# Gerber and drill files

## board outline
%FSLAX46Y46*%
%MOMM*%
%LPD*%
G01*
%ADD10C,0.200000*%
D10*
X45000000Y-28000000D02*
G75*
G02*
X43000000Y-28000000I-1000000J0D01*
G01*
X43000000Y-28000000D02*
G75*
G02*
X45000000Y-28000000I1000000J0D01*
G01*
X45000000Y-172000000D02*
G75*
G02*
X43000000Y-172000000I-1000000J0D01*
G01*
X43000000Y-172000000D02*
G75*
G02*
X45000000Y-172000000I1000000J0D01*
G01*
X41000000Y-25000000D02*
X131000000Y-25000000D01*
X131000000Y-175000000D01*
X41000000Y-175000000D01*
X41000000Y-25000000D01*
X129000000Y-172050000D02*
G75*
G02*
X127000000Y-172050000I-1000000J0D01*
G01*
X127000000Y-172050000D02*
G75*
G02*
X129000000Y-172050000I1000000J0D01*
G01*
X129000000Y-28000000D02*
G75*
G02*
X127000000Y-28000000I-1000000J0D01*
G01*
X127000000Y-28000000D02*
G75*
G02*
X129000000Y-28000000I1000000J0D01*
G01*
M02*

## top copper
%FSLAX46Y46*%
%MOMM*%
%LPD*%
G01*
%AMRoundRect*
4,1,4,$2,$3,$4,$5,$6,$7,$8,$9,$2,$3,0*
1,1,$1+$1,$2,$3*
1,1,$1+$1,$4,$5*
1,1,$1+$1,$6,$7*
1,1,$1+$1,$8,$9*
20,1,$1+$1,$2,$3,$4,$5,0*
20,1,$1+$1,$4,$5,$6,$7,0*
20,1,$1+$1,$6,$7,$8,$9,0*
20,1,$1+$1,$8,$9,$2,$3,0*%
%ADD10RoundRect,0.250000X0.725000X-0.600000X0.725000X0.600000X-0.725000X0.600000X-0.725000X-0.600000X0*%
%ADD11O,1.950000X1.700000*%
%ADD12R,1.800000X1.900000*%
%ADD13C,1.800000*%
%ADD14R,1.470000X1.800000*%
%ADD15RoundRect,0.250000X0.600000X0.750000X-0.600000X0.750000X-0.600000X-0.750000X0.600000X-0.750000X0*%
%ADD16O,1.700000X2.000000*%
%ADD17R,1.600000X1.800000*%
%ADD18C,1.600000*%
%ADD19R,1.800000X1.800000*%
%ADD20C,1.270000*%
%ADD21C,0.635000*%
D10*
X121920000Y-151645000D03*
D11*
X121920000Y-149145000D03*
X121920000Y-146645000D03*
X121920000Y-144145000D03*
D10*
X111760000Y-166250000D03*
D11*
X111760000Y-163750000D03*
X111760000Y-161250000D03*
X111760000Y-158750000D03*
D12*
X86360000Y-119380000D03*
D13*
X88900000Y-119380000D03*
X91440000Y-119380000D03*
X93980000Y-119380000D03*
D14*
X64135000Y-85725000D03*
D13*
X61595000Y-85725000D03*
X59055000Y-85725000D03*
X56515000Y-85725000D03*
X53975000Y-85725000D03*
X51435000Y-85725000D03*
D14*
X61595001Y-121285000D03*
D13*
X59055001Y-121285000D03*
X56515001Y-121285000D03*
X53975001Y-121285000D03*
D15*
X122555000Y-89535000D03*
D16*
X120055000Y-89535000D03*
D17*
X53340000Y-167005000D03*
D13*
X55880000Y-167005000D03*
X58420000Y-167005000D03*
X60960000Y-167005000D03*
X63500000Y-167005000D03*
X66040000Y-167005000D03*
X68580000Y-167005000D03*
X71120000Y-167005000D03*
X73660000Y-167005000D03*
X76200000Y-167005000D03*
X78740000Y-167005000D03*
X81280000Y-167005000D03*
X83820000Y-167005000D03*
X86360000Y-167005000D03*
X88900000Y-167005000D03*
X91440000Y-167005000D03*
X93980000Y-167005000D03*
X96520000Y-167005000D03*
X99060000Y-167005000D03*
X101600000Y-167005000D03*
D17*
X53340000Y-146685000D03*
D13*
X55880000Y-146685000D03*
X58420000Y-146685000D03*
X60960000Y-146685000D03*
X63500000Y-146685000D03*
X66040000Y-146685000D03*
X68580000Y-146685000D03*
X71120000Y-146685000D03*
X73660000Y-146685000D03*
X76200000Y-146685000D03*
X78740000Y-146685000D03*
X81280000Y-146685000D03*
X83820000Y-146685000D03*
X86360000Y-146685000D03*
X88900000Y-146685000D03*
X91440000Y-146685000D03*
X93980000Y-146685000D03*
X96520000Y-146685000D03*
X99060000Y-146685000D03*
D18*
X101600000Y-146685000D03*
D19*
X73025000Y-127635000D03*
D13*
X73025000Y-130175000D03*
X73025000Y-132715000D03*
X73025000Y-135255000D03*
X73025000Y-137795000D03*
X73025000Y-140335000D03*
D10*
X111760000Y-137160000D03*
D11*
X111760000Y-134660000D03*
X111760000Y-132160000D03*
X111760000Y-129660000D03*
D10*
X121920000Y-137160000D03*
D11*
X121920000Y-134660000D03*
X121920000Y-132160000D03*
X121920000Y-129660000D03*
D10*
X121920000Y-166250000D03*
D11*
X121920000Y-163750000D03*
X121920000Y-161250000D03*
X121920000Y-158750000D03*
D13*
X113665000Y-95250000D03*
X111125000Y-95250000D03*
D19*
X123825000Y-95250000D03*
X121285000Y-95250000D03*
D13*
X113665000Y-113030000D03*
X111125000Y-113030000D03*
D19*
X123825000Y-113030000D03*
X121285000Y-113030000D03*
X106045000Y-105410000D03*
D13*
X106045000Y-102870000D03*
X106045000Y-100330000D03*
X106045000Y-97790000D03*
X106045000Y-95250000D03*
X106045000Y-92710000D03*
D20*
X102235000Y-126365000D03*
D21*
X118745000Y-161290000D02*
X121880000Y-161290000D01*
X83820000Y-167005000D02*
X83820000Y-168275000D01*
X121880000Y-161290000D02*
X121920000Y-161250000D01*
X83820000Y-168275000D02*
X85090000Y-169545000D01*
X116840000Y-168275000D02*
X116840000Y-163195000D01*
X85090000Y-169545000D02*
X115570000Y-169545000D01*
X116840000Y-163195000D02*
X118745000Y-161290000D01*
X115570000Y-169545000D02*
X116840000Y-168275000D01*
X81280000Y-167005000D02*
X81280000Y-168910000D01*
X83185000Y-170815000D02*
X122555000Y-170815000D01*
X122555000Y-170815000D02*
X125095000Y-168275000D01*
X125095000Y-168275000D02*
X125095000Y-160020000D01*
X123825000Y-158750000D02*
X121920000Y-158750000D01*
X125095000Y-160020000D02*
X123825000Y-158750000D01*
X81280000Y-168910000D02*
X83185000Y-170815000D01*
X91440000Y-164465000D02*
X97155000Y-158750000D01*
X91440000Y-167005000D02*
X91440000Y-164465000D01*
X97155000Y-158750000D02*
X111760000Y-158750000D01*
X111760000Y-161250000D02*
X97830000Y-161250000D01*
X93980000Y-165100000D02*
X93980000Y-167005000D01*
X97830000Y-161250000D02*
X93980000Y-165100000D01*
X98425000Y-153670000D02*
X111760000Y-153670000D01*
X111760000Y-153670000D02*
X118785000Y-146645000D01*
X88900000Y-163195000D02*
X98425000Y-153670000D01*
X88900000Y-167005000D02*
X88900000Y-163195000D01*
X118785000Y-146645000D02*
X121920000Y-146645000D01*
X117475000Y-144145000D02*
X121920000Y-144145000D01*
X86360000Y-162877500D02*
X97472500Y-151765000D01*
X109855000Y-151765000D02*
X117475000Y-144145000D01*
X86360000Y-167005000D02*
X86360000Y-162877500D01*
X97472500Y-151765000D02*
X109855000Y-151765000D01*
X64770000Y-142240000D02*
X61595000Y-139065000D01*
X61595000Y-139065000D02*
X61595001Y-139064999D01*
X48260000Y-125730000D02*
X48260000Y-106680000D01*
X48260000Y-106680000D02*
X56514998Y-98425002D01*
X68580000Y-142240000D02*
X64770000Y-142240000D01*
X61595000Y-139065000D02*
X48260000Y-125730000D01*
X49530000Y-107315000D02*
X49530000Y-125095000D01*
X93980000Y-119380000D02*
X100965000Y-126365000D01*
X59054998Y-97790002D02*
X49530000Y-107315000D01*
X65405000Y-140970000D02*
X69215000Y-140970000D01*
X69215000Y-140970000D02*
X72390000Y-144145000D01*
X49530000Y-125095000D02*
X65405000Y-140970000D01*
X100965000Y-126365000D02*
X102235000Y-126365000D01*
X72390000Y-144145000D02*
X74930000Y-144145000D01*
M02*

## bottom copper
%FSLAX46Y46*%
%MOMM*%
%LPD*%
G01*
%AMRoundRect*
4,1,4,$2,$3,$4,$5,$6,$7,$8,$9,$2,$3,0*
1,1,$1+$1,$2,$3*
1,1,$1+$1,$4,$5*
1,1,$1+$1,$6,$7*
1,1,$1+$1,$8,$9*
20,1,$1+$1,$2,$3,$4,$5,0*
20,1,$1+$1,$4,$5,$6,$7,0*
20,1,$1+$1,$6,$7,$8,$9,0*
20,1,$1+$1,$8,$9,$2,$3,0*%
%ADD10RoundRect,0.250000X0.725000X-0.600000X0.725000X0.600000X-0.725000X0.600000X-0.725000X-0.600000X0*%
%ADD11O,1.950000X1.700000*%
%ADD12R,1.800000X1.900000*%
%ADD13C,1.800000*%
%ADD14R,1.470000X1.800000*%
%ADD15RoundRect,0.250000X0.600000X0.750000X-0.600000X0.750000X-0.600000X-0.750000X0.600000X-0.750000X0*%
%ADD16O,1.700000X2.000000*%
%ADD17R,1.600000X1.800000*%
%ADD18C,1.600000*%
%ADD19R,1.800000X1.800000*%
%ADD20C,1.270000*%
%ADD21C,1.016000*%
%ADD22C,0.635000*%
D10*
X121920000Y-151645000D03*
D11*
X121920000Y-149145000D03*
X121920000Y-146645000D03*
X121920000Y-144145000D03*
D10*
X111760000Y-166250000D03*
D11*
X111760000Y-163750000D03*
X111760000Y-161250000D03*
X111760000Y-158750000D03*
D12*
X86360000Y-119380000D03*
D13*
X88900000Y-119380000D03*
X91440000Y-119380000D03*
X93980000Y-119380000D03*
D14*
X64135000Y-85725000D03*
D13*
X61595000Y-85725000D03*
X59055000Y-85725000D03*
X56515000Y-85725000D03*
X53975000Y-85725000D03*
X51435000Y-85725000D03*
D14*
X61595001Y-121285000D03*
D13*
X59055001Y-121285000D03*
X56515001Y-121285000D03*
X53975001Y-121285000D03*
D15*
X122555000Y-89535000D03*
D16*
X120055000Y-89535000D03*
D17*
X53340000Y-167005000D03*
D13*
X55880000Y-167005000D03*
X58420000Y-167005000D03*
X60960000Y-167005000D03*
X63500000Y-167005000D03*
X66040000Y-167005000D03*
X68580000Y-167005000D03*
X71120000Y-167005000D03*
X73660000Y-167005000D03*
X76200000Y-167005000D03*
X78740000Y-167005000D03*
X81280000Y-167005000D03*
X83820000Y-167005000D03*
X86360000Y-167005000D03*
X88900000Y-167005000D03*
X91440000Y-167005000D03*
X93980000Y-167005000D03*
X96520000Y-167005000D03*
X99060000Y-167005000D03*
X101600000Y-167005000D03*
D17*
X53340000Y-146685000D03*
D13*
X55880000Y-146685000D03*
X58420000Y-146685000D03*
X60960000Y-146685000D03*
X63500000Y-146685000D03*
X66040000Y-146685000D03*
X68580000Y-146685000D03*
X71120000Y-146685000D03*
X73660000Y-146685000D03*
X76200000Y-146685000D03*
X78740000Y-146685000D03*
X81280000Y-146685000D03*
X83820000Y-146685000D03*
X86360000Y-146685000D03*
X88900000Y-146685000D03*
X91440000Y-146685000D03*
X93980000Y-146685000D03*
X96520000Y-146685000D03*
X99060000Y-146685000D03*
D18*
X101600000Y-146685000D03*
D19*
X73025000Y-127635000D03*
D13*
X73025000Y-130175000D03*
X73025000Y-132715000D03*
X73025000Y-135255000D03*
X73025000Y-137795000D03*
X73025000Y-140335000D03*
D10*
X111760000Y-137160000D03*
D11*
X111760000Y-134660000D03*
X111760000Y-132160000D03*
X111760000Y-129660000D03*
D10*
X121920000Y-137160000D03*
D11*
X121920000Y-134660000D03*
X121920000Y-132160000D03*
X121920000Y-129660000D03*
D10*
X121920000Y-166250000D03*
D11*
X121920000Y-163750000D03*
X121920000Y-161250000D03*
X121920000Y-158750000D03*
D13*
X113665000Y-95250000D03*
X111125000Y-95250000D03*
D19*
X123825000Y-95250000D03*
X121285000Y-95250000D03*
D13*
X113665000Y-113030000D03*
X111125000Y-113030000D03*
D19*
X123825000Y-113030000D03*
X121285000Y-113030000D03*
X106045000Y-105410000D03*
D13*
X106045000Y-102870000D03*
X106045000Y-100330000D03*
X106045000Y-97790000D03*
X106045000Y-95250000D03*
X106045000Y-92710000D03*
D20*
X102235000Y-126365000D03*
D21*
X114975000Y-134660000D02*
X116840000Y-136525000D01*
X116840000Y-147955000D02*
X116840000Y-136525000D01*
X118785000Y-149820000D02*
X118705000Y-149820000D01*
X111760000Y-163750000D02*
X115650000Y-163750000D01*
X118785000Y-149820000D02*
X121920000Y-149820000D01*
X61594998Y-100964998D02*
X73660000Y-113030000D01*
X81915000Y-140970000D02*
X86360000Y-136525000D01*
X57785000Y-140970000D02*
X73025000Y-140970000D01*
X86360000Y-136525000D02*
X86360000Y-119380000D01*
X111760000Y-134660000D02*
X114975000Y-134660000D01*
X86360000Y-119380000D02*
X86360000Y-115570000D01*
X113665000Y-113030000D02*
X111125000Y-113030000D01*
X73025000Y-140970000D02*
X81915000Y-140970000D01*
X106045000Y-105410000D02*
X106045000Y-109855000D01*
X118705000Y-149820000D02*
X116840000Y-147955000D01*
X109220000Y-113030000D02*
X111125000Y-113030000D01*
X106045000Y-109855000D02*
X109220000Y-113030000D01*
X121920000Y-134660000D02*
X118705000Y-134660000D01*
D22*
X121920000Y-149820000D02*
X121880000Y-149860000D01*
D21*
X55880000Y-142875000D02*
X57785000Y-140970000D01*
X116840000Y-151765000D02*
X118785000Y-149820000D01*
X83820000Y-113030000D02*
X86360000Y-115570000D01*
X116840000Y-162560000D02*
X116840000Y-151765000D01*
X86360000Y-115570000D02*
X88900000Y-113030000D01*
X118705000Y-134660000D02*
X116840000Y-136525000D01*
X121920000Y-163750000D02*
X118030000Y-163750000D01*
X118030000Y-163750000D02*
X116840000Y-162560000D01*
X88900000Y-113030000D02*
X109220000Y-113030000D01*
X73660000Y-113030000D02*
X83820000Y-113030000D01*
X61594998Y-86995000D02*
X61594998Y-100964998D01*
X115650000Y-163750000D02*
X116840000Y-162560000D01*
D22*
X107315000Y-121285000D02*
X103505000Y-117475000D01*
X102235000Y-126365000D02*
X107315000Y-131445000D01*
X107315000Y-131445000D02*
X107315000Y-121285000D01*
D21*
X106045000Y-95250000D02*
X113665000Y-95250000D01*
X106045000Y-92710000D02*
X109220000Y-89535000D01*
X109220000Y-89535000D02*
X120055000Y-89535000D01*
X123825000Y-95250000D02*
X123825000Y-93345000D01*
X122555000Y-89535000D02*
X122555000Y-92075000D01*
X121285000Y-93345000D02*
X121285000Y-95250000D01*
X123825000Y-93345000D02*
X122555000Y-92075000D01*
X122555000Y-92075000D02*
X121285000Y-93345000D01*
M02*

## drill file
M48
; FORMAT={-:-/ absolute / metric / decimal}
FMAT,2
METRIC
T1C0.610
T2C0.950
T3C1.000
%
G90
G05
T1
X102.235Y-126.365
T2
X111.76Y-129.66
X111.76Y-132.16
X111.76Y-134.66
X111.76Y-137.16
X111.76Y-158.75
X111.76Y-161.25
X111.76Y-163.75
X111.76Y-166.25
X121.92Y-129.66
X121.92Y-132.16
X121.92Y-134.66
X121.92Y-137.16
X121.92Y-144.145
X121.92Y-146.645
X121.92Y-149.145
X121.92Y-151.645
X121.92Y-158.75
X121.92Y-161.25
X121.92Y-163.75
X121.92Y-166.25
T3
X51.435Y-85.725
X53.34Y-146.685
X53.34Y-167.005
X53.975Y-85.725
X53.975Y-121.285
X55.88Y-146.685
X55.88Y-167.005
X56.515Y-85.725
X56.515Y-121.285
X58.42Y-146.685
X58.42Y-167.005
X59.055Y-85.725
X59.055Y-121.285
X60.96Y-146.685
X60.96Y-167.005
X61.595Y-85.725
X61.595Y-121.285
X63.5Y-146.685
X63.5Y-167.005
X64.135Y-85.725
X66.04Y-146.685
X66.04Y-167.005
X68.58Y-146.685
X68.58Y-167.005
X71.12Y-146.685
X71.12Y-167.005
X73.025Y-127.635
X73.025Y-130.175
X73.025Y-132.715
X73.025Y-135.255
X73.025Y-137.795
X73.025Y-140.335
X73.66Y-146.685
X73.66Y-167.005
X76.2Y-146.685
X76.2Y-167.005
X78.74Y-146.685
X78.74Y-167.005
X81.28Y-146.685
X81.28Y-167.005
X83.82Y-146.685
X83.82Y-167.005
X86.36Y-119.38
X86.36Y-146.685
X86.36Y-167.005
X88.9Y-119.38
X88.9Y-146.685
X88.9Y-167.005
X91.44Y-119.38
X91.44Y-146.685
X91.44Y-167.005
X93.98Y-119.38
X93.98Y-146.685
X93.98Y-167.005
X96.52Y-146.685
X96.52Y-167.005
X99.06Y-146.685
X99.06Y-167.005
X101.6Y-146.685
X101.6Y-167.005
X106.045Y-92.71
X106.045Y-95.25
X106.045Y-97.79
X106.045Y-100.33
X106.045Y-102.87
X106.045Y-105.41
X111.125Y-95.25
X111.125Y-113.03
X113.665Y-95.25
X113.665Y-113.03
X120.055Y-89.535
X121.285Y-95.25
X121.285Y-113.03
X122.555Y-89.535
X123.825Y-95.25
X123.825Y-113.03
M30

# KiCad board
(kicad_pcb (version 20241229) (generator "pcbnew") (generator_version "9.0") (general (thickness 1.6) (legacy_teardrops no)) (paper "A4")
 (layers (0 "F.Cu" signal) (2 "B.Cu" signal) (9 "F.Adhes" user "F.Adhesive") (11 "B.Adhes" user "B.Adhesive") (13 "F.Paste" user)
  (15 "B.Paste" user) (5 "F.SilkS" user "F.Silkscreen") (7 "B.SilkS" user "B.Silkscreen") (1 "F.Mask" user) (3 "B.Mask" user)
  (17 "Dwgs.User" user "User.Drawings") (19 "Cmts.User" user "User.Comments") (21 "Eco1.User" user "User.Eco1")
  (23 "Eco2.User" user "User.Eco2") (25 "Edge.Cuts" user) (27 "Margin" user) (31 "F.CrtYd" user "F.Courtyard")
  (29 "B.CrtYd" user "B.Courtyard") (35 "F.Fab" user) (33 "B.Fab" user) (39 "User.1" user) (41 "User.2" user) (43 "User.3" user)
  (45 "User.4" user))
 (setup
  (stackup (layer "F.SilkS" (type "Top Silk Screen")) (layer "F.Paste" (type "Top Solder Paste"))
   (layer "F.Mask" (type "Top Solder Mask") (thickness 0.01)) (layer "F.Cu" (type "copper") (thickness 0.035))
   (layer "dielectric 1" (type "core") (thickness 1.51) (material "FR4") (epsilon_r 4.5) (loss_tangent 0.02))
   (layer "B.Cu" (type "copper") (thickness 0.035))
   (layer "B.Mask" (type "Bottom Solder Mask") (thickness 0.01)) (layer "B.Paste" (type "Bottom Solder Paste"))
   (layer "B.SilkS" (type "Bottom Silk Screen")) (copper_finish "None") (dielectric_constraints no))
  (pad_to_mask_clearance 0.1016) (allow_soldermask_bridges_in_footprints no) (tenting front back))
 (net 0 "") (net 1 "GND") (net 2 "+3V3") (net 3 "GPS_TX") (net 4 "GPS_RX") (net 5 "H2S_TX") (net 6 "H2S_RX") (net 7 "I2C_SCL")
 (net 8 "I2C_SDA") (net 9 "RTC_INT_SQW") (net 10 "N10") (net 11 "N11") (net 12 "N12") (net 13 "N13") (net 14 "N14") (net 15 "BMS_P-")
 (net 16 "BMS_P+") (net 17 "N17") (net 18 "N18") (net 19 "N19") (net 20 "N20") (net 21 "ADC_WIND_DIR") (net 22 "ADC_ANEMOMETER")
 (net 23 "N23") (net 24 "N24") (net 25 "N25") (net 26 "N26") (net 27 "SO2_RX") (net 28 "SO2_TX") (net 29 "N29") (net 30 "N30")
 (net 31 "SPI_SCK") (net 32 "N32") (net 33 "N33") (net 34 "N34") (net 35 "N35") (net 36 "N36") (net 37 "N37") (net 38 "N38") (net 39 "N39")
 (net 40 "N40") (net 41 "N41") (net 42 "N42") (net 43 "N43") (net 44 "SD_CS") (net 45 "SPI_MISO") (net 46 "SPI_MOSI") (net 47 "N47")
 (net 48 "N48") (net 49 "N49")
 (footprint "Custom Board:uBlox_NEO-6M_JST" (layer "F.Cu") (at 122.01 147.915 90)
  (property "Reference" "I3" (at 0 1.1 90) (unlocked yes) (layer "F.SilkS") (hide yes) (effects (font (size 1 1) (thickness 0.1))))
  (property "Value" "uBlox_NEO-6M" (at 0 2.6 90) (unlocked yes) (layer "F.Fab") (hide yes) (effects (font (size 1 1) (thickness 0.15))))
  (pad "1" thru_hole roundrect (at -3.73 -0.09 90) (size 1.7 1.95) (drill 0.95) (layers "*.Cu" "*.Mask") (remove_unused_layers no)
   (roundrect_rratio 0.147059) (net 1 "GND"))
  (pad "2" thru_hole oval (at -1.23 -0.09 90) (size 1.7 1.95) (drill 0.95) (layers "*.Cu" "*.Mask") (remove_unused_layers no) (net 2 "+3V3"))
  (pad "3" thru_hole oval (at 1.27 -0.09 90) (size 1.7 1.95) (drill 0.95) (layers "*.Cu" "*.Mask") (remove_unused_layers no)
   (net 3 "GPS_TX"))
  (pad "4" thru_hole oval (at 3.77 -0.09 90) (size 1.7 1.95) (drill 0.95) (layers "*.Cu" "*.Mask") (remove_unused_layers no)
   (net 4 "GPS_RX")))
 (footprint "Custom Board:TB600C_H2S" (layer "F.Cu") (at 111.76 162.48 90)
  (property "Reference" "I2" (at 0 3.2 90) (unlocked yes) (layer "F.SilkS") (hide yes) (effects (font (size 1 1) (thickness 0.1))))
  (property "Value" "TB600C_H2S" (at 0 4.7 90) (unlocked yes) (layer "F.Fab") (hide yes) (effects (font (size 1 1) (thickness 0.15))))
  (pad "1" thru_hole roundrect (at -3.77 0 90) (size 1.7 1.95) (drill 0.95) (layers "*.Cu" "*.Mask") (remove_unused_layers no)
   (roundrect_rratio 0.147059) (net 1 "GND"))
  (pad "2" thru_hole oval (at -1.27 0 90) (size 1.7 1.95) (drill 0.95) (layers "*.Cu" "*.Mask") (remove_unused_layers no) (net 2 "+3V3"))
  (pad "3" thru_hole oval (at 1.23 0 90) (size 1.7 1.95) (drill 0.95) (layers "*.Cu" "*.Mask") (remove_unused_layers no) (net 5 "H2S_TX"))
  (pad "4" thru_hole oval (at 3.73 0 90) (size 1.7 1.95) (drill 0.95) (layers "*.Cu" "*.Mask") (remove_unused_layers no) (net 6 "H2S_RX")))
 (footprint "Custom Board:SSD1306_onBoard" (layer "F.Cu") (at 90.17 130.81)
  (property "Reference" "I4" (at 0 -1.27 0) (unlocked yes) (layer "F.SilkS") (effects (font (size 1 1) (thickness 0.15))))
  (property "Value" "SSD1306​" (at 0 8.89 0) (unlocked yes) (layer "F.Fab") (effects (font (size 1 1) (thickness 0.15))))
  (pad "1" thru_hole rect (at -3.81 -11.43) (size 1.8 1.9) (drill 1) (layers "*.Cu" "*.Mask") (remove_unused_layers no) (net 2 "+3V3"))
  (pad "2" thru_hole circle (at -1.27 -11.43) (size 1.8 1.8) (drill 1) (layers "*.Cu" "*.Mask") (remove_unused_layers no) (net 1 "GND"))
  (pad "3" thru_hole circle (at 1.27 -11.43) (size 1.8 1.8) (drill 1) (layers "*.Cu" "*.Mask") (remove_unused_layers no) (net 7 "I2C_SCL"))
  (pad "4" thru_hole circle (at 3.81 -11.43) (size 1.8 1.8) (drill 1) (layers "*.Cu" "*.Mask") (remove_unused_layers no) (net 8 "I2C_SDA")))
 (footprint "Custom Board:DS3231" (layer "F.Cu") (at 59.055001 103.505 90)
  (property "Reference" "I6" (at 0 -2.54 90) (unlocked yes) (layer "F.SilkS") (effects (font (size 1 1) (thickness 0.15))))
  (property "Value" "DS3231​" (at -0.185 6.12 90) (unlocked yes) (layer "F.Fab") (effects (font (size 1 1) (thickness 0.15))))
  (pad "1" thru_hole rect (at 17.78 5.079999 270) (size 1.8 1.47) (drill 1) (layers "*.Cu" "*.Mask") (remove_unused_layers no) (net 1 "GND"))
  (pad "2" thru_hole circle (at 17.78 2.539999 270) (size 1.8 1.8) (drill 1) (layers "*.Cu" "*.Mask") (remove_unused_layers no)
   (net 2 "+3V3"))
  (pad "3" thru_hole circle (at 17.78 -0.000001 270) (size 1.8 1.8) (drill 1) (layers "*.Cu" "*.Mask") (remove_unused_layers no)
   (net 8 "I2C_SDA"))
  (pad "4" thru_hole circle (at 17.78 -2.540001 270) (size 1.8 1.8) (drill 1) (layers "*.Cu" "*.Mask") (remove_unused_layers no)
   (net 7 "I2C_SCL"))
  (pad "5" thru_hole circle (at 17.78 -5.080001 270) (size 1.8 1.8) (drill 1) (layers "*.Cu" "*.Mask") (remove_unused_layers no)
   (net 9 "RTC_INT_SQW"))
  (pad "6" thru_hole circle (at 17.78 -7.620001 270) (size 1.8 1.8) (drill 1) (layers "*.Cu" "*.Mask") (remove_unused_layers no)
   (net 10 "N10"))
  (pad "7" thru_hole rect (at -17.78 2.54 270) (size 1.8 1.47) (drill 1) (layers "*.Cu" "*.Mask") (remove_unused_layers no) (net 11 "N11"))
  (pad "8" thru_hole circle (at -17.78 0 270) (size 1.8 1.8) (drill 1) (layers "*.Cu" "*.Mask") (remove_unused_layers no) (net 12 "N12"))
  (pad "9" thru_hole circle (at -17.78 -2.54 270) (size 1.8 1.8) (drill 1) (layers "*.Cu" "*.Mask") (remove_unused_layers no) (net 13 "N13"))
  (pad "10" thru_hole circle (at -17.78 -5.08 270) (size 1.8 1.8) (drill 1) (layers "*.Cu" "*.Mask") (remove_unused_layers no)
   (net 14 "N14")))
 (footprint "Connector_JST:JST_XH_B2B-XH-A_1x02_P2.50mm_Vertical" (layer "F.Cu") (at 122.555 89.535 180)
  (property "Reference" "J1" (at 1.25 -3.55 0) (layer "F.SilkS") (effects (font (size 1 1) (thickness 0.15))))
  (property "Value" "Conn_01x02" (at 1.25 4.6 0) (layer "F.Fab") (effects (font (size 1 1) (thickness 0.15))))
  (pad "1" thru_hole roundrect (at 0 0 180) (size 1.7 2) (drill 1) (layers "*.Cu" "*.Mask") (remove_unused_layers no)
   (roundrect_rratio 0.147059) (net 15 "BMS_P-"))
  (pad "2" thru_hole oval (at 2.5 0 180) (size 1.7 2) (drill 1) (layers "*.Cu" "*.Mask") (remove_unused_layers no) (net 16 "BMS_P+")))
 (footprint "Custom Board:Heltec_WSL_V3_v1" (layer "F.Cu") (at 73.66 156.845 -90)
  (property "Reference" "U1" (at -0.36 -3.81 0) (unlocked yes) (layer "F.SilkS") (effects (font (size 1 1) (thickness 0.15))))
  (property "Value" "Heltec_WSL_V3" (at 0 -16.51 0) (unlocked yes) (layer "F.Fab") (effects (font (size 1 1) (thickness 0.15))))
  (pad "1" thru_hole rect (at 10.16 20.32 270) (size 1.8 1.6) (drill 1) (layers "*.Cu" "*.Mask") (remove_unused_layers no) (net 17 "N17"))
  (pad "2" thru_hole circle (at 10.16 17.78 180) (size 1.8 1.8) (drill 1) (layers "*.Cu" "*.Mask") (remove_unused_layers no) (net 1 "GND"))
  (pad "3" thru_hole circle (at 10.16 15.24 180) (size 1.8 1.8) (drill 1) (layers "*.Cu" "*.Mask") (remove_unused_layers no) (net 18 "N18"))
  (pad "4" thru_hole circle (at 10.16 12.7 180) (size 1.8 1.8) (drill 1) (layers "*.Cu" "*.Mask") (remove_unused_layers no) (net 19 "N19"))
  (pad "5" thru_hole circle (at 10.16 10.16 180) (size 1.8 1.8) (drill 1) (layers "*.Cu" "*.Mask") (remove_unused_layers no) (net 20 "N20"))
  (pad "6" thru_hole circle (at 10.16 7.62 180) (size 1.8 1.8) (drill 1) (layers "*.Cu" "*.Mask") (remove_unused_layers no)
   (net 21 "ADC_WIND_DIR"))
  (pad "7" thru_hole circle (at 10.16 5.08 180) (size 1.8 1.8) (drill 1) (layers "*.Cu" "*.Mask") (remove_unused_layers no)
   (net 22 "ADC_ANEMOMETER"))
  (pad "8" thru_hole circle (at 10.16 2.54 180) (size 1.8 1.8) (drill 1) (layers "*.Cu" "*.Mask") (remove_unused_layers no) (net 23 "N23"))
  (pad "9" thru_hole circle (at 10.16 0 180) (size 1.8 1.8) (drill 1) (layers "*.Cu" "*.Mask") (remove_unused_layers no) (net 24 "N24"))
  (pad "10" thru_hole circle (at 10.16 -2.54 180) (size 1.8 1.8) (drill 1) (layers "*.Cu" "*.Mask") (remove_unused_layers no) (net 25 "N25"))
  (pad "11" thru_hole circle (at 10.16 -5.08 180) (size 1.8 1.8) (drill 1) (layers "*.Cu" "*.Mask") (remove_unused_layers no) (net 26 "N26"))
  (pad "12" thru_hole circle (at 10.16 -7.62 180) (size 1.8 1.8) (drill 1) (layers "*.Cu" "*.Mask") (remove_unused_layers no)
   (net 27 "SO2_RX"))
  (pad "13" thru_hole circle (at 10.16 -10.16 180) (size 1.8 1.8) (drill 1) (layers "*.Cu" "*.Mask") (remove_unused_layers no)
   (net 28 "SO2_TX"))
  (pad "14" thru_hole circle (at 10.16 -12.7 180) (size 1.8 1.8) (drill 1) (layers "*.Cu" "*.Mask") (remove_unused_layers no)
   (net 4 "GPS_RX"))
  (pad "15" thru_hole circle (at 10.16 -15.24 180) (size 1.8 1.8) (drill 1) (layers "*.Cu" "*.Mask") (remove_unused_layers no)
   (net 3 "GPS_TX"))
  (pad "16" thru_hole circle (at 10.16 -17.78 180) (size 1.8 1.8) (drill 1) (layers "*.Cu" "*.Mask") (remove_unused_layers no)
   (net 6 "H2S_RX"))
  (pad "17" thru_hole circle (at 10.16 -20.32 180) (size 1.8 1.8) (drill 1) (layers "*.Cu" "*.Mask") (remove_unused_layers no)
   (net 5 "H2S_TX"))
  (pad "18" thru_hole circle (at 10.16 -22.86 180) (size 1.8 1.8) (drill 1) (layers "*.Cu" "*.Mask") (remove_unused_layers no)
   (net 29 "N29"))
  (pad "19" thru_hole circle (at 10.16 -25.4 180) (size 1.8 1.8) (drill 1) (layers "*.Cu" "*.Mask") (remove_unused_layers no) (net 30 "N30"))
  (pad "20" thru_hole circle (at 10.16 -27.94 180) (size 1.8 1.8) (drill 1) (layers "*.Cu" "*.Mask") (remove_unused_layers no)
   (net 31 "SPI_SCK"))
  (pad "21" thru_hole rect (at -10.16 20.32 270) (size 1.8 1.6) (drill 1) (layers "*.Cu" "*.Mask") (remove_unused_layers no) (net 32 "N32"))
  (pad "22" thru_hole circle (at -10.16 17.78 180) (size 1.8 1.8) (drill 1) (layers "*.Cu" "*.Mask") (remove_unused_layers no)
   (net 2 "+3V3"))
  (pad "23" thru_hole circle (at -10.16 15.24 180) (size 1.8 1.8) (drill 1) (layers "*.Cu" "*.Mask") (remove_unused_layers no) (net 1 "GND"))
  (pad "24" thru_hole circle (at -10.16 12.7 180) (size 1.8 1.8) (drill 1) (layers "*.Cu" "*.Mask") (remove_unused_layers no) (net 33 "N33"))
  (pad "25" thru_hole circle (at -10.16 10.16 180) (size 1.8 1.8) (drill 1) (layers "*.Cu" "*.Mask") (remove_unused_layers no)
   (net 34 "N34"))
  (pad "26" thru_hole circle (at -10.16 7.62 180) (size 1.8 1.8) (drill 1) (layers "*.Cu" "*.Mask") (remove_unused_layers no) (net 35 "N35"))
  (pad "27" thru_hole circle (at -10.16 5.08 180) (size 1.8 1.8) (drill 1) (layers "*.Cu" "*.Mask") (remove_unused_layers no) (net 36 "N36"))
  (pad "28" thru_hole circle (at -10.16 2.54 180) (size 1.8 1.8) (drill 1) (layers "*.Cu" "*.Mask") (remove_unused_layers no)
   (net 7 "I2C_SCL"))
  (pad "29" thru_hole circle (at -10.16 0 180) (size 1.8 1.8) (drill 1) (layers "*.Cu" "*.Mask") (remove_unused_layers no) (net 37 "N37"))
  (pad "30" thru_hole circle (at -10.16 -2.54 180) (size 1.8 1.8) (drill 1) (layers "*.Cu" "*.Mask") (remove_unused_layers no)
   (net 8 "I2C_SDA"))
  (pad "31" thru_hole circle (at -10.16 -5.08 180) (size 1.8 1.8) (drill 1) (layers "*.Cu" "*.Mask") (remove_unused_layers no)
   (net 9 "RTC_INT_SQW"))
  (pad "32" thru_hole circle (at -10.16 -7.62 180) (size 1.8 1.8) (drill 1) (layers "*.Cu" "*.Mask") (remove_unused_layers no)
   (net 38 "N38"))
  (pad "33" thru_hole circle (at -10.16 -10.16 180) (size 1.8 1.8) (drill 1) (layers "*.Cu" "*.Mask") (remove_unused_layers no)
   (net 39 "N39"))
  (pad "34" thru_hole circle (at -10.16 -12.7 180) (size 1.8 1.8) (drill 1) (layers "*.Cu" "*.Mask") (remove_unused_layers no)
   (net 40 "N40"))
  (pad "35" thru_hole circle (at -10.16 -15.24 180) (size 1.8 1.8) (drill 1) (layers "*.Cu" "*.Mask") (remove_unused_layers no)
   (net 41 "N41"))
  (pad "36" thru_hole circle (at -10.16 -17.78 180) (size 1.8 1.8) (drill 1) (layers "*.Cu" "*.Mask") (remove_unused_layers no)
   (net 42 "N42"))
  (pad "37" thru_hole circle (at -10.16 -20.32 180) (size 1.8 1.8) (drill 1) (layers "*.Cu" "*.Mask") (remove_unused_layers no)
   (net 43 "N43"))
  (pad "38" thru_hole circle (at -10.16 -22.86 180) (size 1.8 1.8) (drill 1) (layers "*.Cu" "*.Mask") (remove_unused_layers no)
   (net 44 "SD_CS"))
  (pad "39" thru_hole circle (at -10.16 -25.4 180) (size 1.8 1.8) (drill 1) (layers "*.Cu" "*.Mask") (remove_unused_layers no)
   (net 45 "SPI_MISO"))
  (pad "40" thru_hole circle (at -10.16 -27.94 180) (size 1.6 1.6) (drill 1) (layers "*.Cu" "*.Mask") (remove_unused_layers no)
   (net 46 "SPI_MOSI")))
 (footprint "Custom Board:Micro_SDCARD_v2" (layer "F.Cu") (at 60.325 133.985)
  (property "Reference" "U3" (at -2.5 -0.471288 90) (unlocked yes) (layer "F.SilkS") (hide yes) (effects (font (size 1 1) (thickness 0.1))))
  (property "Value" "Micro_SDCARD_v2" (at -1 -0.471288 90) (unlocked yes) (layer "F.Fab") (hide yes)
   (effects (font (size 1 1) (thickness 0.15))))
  (pad "1" thru_hole rect (at 12.7 -6.35 270) (size 1.8 1.8) (drill 1) (layers "*.Cu" "*.Mask") (remove_unused_layers no) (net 1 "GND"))
  (pad "2" thru_hole circle (at 12.7 -3.81 270) (size 1.8 1.8) (drill 1) (layers "*.Cu" "*.Mask") (remove_unused_layers no)
   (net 45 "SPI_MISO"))
  (pad "3" thru_hole circle (at 12.7 -1.27 270) (size 1.8 1.8) (drill 1) (layers "*.Cu" "*.Mask") (remove_unused_layers no)
   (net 31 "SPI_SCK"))
  (pad "4" thru_hole circle (at 12.7 1.27 270) (size 1.8 1.8) (drill 1) (layers "*.Cu" "*.Mask") (remove_unused_layers no)
   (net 46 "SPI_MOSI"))
  (pad "5" thru_hole circle (at 12.7 3.81 270) (size 1.8 1.8) (drill 1) (layers "*.Cu" "*.Mask") (remove_unused_layers no) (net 44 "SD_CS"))
  (pad "6" thru_hole circle (at 12.7 6.35 270) (size 1.8 1.8) (drill 1) (layers "*.Cu" "*.Mask") (remove_unused_layers no) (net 2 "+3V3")))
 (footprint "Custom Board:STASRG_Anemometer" (layer "F.Cu") (at 111.76 133.41 90)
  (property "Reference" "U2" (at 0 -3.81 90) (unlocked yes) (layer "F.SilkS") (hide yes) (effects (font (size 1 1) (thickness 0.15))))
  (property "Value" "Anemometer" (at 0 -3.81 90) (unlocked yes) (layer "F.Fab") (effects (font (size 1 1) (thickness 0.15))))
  (pad "1" thru_hole roundrect (at -3.75 0 90) (size 1.7 1.95) (drill 0.95) (layers "*.Cu" "*.Mask") (remove_unused_layers no)
   (roundrect_rratio 0.147059) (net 1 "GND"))
  (pad "2" thru_hole oval (at -1.25 0 90) (size 1.7 1.95) (drill 0.95) (layers "*.Cu" "*.Mask") (remove_unused_layers no) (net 2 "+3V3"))
  (pad "3" thru_hole oval (at 1.25 0 90) (size 1.7 1.95) (drill 0.95) (layers "*.Cu" "*.Mask") (remove_unused_layers no)
   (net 22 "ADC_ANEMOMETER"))
  (pad "4" thru_hole oval (at 3.75 0 90) (size 1.7 1.95) (drill 0.95) (layers "*.Cu" "*.Mask") (remove_unused_layers no) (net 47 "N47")))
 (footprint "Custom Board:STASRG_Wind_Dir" (layer "F.Cu") (at 121.92 133.41 90)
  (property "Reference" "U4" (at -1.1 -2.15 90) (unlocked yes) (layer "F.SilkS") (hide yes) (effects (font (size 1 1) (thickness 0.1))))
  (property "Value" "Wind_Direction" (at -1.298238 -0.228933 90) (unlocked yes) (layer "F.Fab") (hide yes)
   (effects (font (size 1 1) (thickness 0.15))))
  (pad "1" thru_hole roundrect (at -3.75 0 90) (size 1.7 1.95) (drill 0.95) (layers "*.Cu" "*.Mask") (remove_unused_layers no)
   (roundrect_rratio 0.147059) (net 1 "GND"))
  (pad "2" thru_hole oval (at -1.25 0 90) (size 1.7 1.95) (drill 0.95) (layers "*.Cu" "*.Mask") (remove_unused_layers no) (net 2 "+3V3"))
  (pad "3" thru_hole oval (at 1.25 0 90) (size 1.7 1.95) (drill 0.95) (layers "*.Cu" "*.Mask") (remove_unused_layers no)
   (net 21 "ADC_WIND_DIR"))
  (pad "4" thru_hole oval (at 3.75 0 90) (size 1.7 1.95) (drill 0.95) (layers "*.Cu" "*.Mask") (remove_unused_layers no) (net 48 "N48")))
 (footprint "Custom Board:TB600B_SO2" (layer "F.Cu") (at 121.92 162.56 90)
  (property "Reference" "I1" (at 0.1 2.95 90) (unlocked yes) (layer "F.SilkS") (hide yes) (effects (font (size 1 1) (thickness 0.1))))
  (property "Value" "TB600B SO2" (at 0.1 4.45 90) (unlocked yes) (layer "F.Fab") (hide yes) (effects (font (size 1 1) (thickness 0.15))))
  (pad "1" thru_hole roundrect (at -3.69 0 90) (size 1.7 1.95) (drill 0.95) (layers "*.Cu" "*.Mask") (remove_unused_layers no)
   (roundrect_rratio 0.147059) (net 1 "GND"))
  (pad "2" thru_hole oval (at -1.19 0 90) (size 1.7 1.95) (drill 0.95) (layers "*.Cu" "*.Mask") (remove_unused_layers no) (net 2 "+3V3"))
  (pad "3" thru_hole oval (at 1.31 0 90) (size 1.7 1.95) (drill 0.95) (layers "*.Cu" "*.Mask") (remove_unused_layers no) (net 28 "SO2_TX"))
  (pad "4" thru_hole oval (at 3.81 0 90) (size 1.7 1.95) (drill 0.95) (layers "*.Cu" "*.Mask") (remove_unused_layers no) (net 27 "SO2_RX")))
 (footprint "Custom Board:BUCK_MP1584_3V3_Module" (layer "F.Cu") (at 117.475 104.14 -90)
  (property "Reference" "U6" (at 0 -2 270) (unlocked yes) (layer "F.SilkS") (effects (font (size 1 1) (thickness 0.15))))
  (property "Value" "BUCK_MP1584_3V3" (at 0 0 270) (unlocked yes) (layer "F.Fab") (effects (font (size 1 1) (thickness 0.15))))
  (pad "1" thru_hole circle (at -8.89 3.81 270) (size 1.8 1.8) (drill 1) (layers "*.Cu" "*.Mask") (remove_unused_layers no) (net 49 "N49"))
  (pad "1" thru_hole circle (at -8.89 6.35 270) (size 1.8 1.8) (drill 1) (layers "*.Cu" "*.Mask") (remove_unused_layers no) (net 49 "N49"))
  (pad "2" thru_hole rect (at -8.89 -6.35 270) (size 1.8 1.8) (drill 1) (layers "*.Cu" "*.Mask") (remove_unused_layers no) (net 15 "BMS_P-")
   (thermal_bridge_angle 45))
  (pad "2" thru_hole rect (at -8.89 -3.81 270) (size 1.8 1.8) (drill 1) (layers "*.Cu" "*.Mask") (remove_unused_layers no) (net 15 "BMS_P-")
   (thermal_bridge_angle 45))
  (pad "3" thru_hole circle (at 8.89 3.81 270) (size 1.8 1.8) (drill 1) (layers "*.Cu" "*.Mask") (remove_unused_layers no) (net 2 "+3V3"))
  (pad "3" thru_hole circle (at 8.89 6.35 270) (size 1.8 1.8) (drill 1) (layers "*.Cu" "*.Mask") (remove_unused_layers no) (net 2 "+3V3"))
  (pad "4" thru_hole rect (at 8.89 -6.35 270) (size 1.8 1.8) (drill 1) (layers "*.Cu" "*.Mask") (remove_unused_layers no) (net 1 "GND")
   (thermal_bridge_angle 45))
  (pad "4" thru_hole rect (at 8.89 -3.81 270) (size 1.8 1.8) (drill 1) (layers "*.Cu" "*.Mask") (remove_unused_layers no) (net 1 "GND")
   (thermal_bridge_angle 45)))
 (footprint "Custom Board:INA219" (layer "F.Cu") (at 97.155 99.06)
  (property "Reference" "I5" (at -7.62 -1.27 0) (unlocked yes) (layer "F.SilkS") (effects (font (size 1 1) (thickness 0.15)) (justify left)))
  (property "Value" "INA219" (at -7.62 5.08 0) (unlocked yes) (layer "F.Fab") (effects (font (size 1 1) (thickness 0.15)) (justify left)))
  (pad "1" thru_hole rect (at 8.89 6.35 90) (size 1.8 1.8) (drill 1) (layers "*.Cu" "*.Mask") (remove_unused_layers no) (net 2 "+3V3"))
  (pad "2" thru_hole circle (at 8.89 3.81 90) (size 1.8 1.8) (drill 1) (layers "*.Cu" "*.Mask") (remove_unused_layers no) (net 1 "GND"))
  (pad "3" thru_hole circle (at 8.89 1.27 90) (size 1.8 1.8) (drill 1) (layers "*.Cu" "*.Mask") (remove_unused_layers no) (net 7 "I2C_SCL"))
  (pad "4" thru_hole circle (at 8.89 -1.27 90) (size 1.8 1.8) (drill 1) (layers "*.Cu" "*.Mask") (remove_unused_layers no) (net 8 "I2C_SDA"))
  (pad "5" thru_hole circle (at 8.89 -3.81 90) (size 1.8 1.8) (drill 1) (layers "*.Cu" "*.Mask") (remove_unused_layers no) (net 49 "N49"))
  (pad "6" thru_hole circle (at 8.89 -6.35 90) (size 1.8 1.8) (drill 1) (layers "*.Cu" "*.Mask") (remove_unused_layers no) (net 16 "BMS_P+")))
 (gr_circle (center 44 28) (end 45 28) (stroke (width 0.2) (type default)) (fill no) (layer "Edge.Cuts"))
 (gr_circle (center 44 172) (end 45 172) (stroke (width 0.2) (type default)) (fill no) (layer "Edge.Cuts"))
 (gr_rect (start 41 25) (end 131 175) (stroke (width 0.2) (type default)) (fill no) (layer "Edge.Cuts"))
 (gr_circle (center 128 172.05) (end 129 172.05) (stroke (width 0.2) (type default)) (fill no) (layer "Edge.Cuts"))
 (gr_circle (center 128 28) (end 129 28) (stroke (width 0.2) (type default)) (fill no) (layer "Edge.Cuts"))
 (segment (start 114.975 134.66) (end 116.84 136.525) (width 1.016) (layer "B.Cu") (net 2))
 (segment (start 116.84 147.955) (end 116.84 136.525) (width 1.016) (layer "B.Cu") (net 2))
 (segment (start 118.785 149.82) (end 118.705 149.82) (width 1.016) (layer "B.Cu") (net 2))
 (segment (start 111.76 163.75) (end 115.65 163.75) (width 1.016) (layer "B.Cu") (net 2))
 (segment (start 118.785 149.82) (end 121.92 149.82) (width 1.016) (layer "B.Cu") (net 2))
 (segment (start 61.594998 100.964998) (end 73.66 113.03) (width 1.016) (layer "B.Cu") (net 2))
 (segment (start 81.915 140.97) (end 86.36 136.525) (width 1.016) (layer "B.Cu") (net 2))
 (segment (start 57.785 140.97) (end 73.025 140.97) (width 1.016) (layer "B.Cu") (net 2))
 (segment (start 86.36 136.525) (end 86.36 119.38) (width 1.016) (layer "B.Cu") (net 2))
 (segment (start 111.76 134.66) (end 114.975 134.66) (width 1.016) (layer "B.Cu") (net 2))
 (segment (start 86.36 119.38) (end 86.36 115.57) (width 1.016) (layer "B.Cu") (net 2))
 (segment (start 113.665 113.03) (end 111.125 113.03) (width 1.016) (layer "B.Cu") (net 2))
 (segment (start 73.025 140.97) (end 81.915 140.97) (width 1.016) (layer "B.Cu") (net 2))
 (segment (start 106.045 105.41) (end 106.045 109.855) (width 1.016) (layer "B.Cu") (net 2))
 (segment (start 118.705 149.82) (end 116.84 147.955) (width 1.016) (layer "B.Cu") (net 2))
 (segment (start 109.22 113.03) (end 111.125 113.03) (width 1.016) (layer "B.Cu") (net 2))
 (segment (start 106.045 109.855) (end 109.22 113.03) (width 1.016) (layer "B.Cu") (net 2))
 (segment (start 121.92 134.66) (end 118.705 134.66) (width 1.016) (layer "B.Cu") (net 2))
 (segment (start 121.92 149.82) (end 121.88 149.86) (width 0.635) (layer "B.Cu") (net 2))
 (segment (start 55.88 142.875) (end 57.785 140.97) (width 1.016) (layer "B.Cu") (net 2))
 (segment (start 116.84 151.765) (end 118.785 149.82) (width 1.016) (layer "B.Cu") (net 2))
 (segment (start 83.82 113.03) (end 86.36 115.57) (width 1.016) (layer "B.Cu") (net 2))
 (segment (start 116.84 162.56) (end 116.84 151.765) (width 1.016) (layer "B.Cu") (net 2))
 (segment (start 86.36 115.57) (end 88.9 113.03) (width 1.016) (layer "B.Cu") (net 2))
 (segment (start 118.705 134.66) (end 116.84 136.525) (width 1.016) (layer "B.Cu") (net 2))
 (segment (start 121.92 163.75) (end 118.03 163.75) (width 1.016) (layer "B.Cu") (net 2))
 (segment (start 118.03 163.75) (end 116.84 162.56) (width 1.016) (layer "B.Cu") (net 2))
 (segment (start 88.9 113.03) (end 109.22 113.03) (width 1.016) (layer "B.Cu") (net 2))
 (segment (start 73.66 113.03) (end 83.82 113.03) (width 1.016) (layer "B.Cu") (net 2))
 (segment (start 61.594998 86.995) (end 61.594998 100.964998) (width 1.016) (layer "B.Cu") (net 2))
 (segment (start 115.65 163.75) (end 116.84 162.56) (width 1.016) (layer "B.Cu") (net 2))
 (segment (start 118.745 161.29) (end 121.88 161.29) (width 0.635) (layer "F.Cu") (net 28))
 (segment (start 83.82 167.005) (end 83.82 168.275) (width 0.635) (layer "F.Cu") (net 28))
 (segment (start 121.88 161.29) (end 121.92 161.25) (width 0.635) (layer "F.Cu") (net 28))
 (segment (start 83.82 168.275) (end 85.09 169.545) (width 0.635) (layer "F.Cu") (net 28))
 (segment (start 116.84 168.275) (end 116.84 163.195) (width 0.635) (layer "F.Cu") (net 28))
 (segment (start 85.09 169.545) (end 115.57 169.545) (width 0.635) (layer "F.Cu") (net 28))
 (segment (start 116.84 163.195) (end 118.745 161.29) (width 0.635) (layer "F.Cu") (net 28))
 (segment (start 115.57 169.545) (end 116.84 168.275) (width 0.635) (layer "F.Cu") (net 28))
 (segment (start 81.28 167.005) (end 81.28 168.91) (width 0.635) (layer "F.Cu") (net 27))
 (segment (start 83.185 170.815) (end 122.555 170.815) (width 0.635) (layer "F.Cu") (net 27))
 (segment (start 122.555 170.815) (end 125.095 168.275) (width 0.635) (layer "F.Cu") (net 27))
 (segment (start 125.095 168.275) (end 125.095 160.02) (width 0.635) (layer "F.Cu") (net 27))
 (segment (start 123.825 158.75) (end 121.92 158.75) (width 0.635) (layer "F.Cu") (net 27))
 (segment (start 125.095 160.02) (end 123.825 158.75) (width 0.635) (layer "F.Cu") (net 27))
 (segment (start 81.28 168.91) (end 83.185 170.815) (width 0.635) (layer "F.Cu") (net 27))
 (segment (start 91.44 164.465) (end 97.155 158.75) (width 0.635) (layer "F.Cu") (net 6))
 (segment (start 91.44 167.005) (end 91.44 164.465) (width 0.635) (layer "F.Cu") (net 6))
 (segment (start 97.155 158.75) (end 111.76 158.75) (width 0.635) (layer "F.Cu") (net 6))
 (segment (start 111.76 161.25) (end 97.83 161.25) (width 0.635) (layer "F.Cu") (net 5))
 (segment (start 93.98 165.1) (end 93.98 167.005) (width 0.635) (layer "F.Cu") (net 5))
 (segment (start 97.83 161.25) (end 93.98 165.1) (width 0.635) (layer "F.Cu") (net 5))
 (segment (start 98.425 153.67) (end 111.76 153.67) (width 0.635) (layer "F.Cu") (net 3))
 (segment (start 111.76 153.67) (end 118.785 146.645) (width 0.635) (layer "F.Cu") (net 3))
 (segment (start 88.9 163.195) (end 98.425 153.67) (width 0.635) (layer "F.Cu") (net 3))
 (segment (start 88.9 167.005) (end 88.9 163.195) (width 0.635) (layer "F.Cu") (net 3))
 (segment (start 118.785 146.645) (end 121.92 146.645) (width 0.635) (layer "F.Cu") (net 3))
 (segment (start 117.475 144.145) (end 121.92 144.145) (width 0.635) (layer "F.Cu") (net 4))
 (segment (start 86.36 162.8775) (end 97.4725 151.765) (width 0.635) (layer "F.Cu") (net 4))
 (segment (start 109.855 151.765) (end 117.475 144.145) (width 0.635) (layer "F.Cu") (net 4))
 (segment (start 86.36 167.005) (end 86.36 162.8775) (width 0.635) (layer "F.Cu") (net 4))
 (segment (start 97.4725 151.765) (end 109.855 151.765) (width 0.635) (layer "F.Cu") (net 4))
 (segment (start 64.77 142.24) (end 61.595 139.065) (width 0.635) (layer "F.Cu") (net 7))
 (segment (start 61.595 139.065) (end 61.595001 139.064999) (width 0.635) (layer "F.Cu") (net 7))
 (segment (start 48.26 125.73) (end 48.26 106.68) (width 0.635) (layer "F.Cu") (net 7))
 (segment (start 48.26 106.68) (end 56.514998 98.425002) (width 0.635) (layer "F.Cu") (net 7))
 (segment (start 68.58 142.24) (end 64.77 142.24) (width 0.635) (layer "F.Cu") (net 7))
 (segment (start 61.595 139.065) (end 48.26 125.73) (width 0.635) (layer "F.Cu") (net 7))
 (segment (start 49.53 107.315) (end 49.53 125.095) (width 0.635) (layer "F.Cu") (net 8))
 (segment (start 93.98 119.38) (end 100.965 126.365) (width 0.635) (layer "F.Cu") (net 8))
 (segment (start 59.054998 97.790002) (end 49.53 107.315) (width 0.635) (layer "F.Cu") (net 8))
 (segment (start 65.405 140.97) (end 69.215 140.97) (width 0.635) (layer "F.Cu") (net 8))
 (segment (start 69.215 140.97) (end 72.39 144.145) (width 0.635) (layer "F.Cu") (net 8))
 (segment (start 49.53 125.095) (end 65.405 140.97) (width 0.635) (layer "F.Cu") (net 8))
 (segment (start 100.965 126.365) (end 102.235 126.365) (width 0.635) (layer "F.Cu") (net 8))
 (segment (start 72.39 144.145) (end 74.93 144.145) (width 0.635) (layer "F.Cu") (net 8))
 (via (at 102.235 126.365) (size 1.27) (drill 0.6096) (layers "F.Cu" "B.Cu") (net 8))
 (segment (start 107.315 121.285) (end 103.505 117.475) (width 0.635) (layer "B.Cu") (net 8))
 (segment (start 102.235 126.365) (end 107.315 131.445) (width 0.635) (layer "B.Cu") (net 8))
 (segment (start 107.315 131.445) (end 107.315 121.285) (width 0.635) (layer "B.Cu") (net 8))
 (segment (start 106.045 95.25) (end 113.665 95.25) (width 1.016) (layer "B.Cu") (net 49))
 (segment (start 106.045 92.71) (end 109.22 89.535) (width 1.016) (layer "B.Cu") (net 16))
 (segment (start 109.22 89.535) (end 120.055 89.535) (width 1.016) (layer "B.Cu") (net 16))
 (segment (start 123.825 95.25) (end 123.825 93.345) (width 1.016) (layer "B.Cu") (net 15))
 (segment (start 122.555 89.535) (end 122.555 92.075) (width 1.016) (layer "B.Cu") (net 15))
 (segment (start 121.285 93.345) (end 121.285 95.25) (width 1.016) (layer "B.Cu") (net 15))
 (segment (start 123.825 93.345) (end 122.555 92.075) (width 1.016) (layer "B.Cu") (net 15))
 (segment (start 122.555 92.075) (end 121.285 93.345) (width 1.016) (layer "B.Cu") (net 15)))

